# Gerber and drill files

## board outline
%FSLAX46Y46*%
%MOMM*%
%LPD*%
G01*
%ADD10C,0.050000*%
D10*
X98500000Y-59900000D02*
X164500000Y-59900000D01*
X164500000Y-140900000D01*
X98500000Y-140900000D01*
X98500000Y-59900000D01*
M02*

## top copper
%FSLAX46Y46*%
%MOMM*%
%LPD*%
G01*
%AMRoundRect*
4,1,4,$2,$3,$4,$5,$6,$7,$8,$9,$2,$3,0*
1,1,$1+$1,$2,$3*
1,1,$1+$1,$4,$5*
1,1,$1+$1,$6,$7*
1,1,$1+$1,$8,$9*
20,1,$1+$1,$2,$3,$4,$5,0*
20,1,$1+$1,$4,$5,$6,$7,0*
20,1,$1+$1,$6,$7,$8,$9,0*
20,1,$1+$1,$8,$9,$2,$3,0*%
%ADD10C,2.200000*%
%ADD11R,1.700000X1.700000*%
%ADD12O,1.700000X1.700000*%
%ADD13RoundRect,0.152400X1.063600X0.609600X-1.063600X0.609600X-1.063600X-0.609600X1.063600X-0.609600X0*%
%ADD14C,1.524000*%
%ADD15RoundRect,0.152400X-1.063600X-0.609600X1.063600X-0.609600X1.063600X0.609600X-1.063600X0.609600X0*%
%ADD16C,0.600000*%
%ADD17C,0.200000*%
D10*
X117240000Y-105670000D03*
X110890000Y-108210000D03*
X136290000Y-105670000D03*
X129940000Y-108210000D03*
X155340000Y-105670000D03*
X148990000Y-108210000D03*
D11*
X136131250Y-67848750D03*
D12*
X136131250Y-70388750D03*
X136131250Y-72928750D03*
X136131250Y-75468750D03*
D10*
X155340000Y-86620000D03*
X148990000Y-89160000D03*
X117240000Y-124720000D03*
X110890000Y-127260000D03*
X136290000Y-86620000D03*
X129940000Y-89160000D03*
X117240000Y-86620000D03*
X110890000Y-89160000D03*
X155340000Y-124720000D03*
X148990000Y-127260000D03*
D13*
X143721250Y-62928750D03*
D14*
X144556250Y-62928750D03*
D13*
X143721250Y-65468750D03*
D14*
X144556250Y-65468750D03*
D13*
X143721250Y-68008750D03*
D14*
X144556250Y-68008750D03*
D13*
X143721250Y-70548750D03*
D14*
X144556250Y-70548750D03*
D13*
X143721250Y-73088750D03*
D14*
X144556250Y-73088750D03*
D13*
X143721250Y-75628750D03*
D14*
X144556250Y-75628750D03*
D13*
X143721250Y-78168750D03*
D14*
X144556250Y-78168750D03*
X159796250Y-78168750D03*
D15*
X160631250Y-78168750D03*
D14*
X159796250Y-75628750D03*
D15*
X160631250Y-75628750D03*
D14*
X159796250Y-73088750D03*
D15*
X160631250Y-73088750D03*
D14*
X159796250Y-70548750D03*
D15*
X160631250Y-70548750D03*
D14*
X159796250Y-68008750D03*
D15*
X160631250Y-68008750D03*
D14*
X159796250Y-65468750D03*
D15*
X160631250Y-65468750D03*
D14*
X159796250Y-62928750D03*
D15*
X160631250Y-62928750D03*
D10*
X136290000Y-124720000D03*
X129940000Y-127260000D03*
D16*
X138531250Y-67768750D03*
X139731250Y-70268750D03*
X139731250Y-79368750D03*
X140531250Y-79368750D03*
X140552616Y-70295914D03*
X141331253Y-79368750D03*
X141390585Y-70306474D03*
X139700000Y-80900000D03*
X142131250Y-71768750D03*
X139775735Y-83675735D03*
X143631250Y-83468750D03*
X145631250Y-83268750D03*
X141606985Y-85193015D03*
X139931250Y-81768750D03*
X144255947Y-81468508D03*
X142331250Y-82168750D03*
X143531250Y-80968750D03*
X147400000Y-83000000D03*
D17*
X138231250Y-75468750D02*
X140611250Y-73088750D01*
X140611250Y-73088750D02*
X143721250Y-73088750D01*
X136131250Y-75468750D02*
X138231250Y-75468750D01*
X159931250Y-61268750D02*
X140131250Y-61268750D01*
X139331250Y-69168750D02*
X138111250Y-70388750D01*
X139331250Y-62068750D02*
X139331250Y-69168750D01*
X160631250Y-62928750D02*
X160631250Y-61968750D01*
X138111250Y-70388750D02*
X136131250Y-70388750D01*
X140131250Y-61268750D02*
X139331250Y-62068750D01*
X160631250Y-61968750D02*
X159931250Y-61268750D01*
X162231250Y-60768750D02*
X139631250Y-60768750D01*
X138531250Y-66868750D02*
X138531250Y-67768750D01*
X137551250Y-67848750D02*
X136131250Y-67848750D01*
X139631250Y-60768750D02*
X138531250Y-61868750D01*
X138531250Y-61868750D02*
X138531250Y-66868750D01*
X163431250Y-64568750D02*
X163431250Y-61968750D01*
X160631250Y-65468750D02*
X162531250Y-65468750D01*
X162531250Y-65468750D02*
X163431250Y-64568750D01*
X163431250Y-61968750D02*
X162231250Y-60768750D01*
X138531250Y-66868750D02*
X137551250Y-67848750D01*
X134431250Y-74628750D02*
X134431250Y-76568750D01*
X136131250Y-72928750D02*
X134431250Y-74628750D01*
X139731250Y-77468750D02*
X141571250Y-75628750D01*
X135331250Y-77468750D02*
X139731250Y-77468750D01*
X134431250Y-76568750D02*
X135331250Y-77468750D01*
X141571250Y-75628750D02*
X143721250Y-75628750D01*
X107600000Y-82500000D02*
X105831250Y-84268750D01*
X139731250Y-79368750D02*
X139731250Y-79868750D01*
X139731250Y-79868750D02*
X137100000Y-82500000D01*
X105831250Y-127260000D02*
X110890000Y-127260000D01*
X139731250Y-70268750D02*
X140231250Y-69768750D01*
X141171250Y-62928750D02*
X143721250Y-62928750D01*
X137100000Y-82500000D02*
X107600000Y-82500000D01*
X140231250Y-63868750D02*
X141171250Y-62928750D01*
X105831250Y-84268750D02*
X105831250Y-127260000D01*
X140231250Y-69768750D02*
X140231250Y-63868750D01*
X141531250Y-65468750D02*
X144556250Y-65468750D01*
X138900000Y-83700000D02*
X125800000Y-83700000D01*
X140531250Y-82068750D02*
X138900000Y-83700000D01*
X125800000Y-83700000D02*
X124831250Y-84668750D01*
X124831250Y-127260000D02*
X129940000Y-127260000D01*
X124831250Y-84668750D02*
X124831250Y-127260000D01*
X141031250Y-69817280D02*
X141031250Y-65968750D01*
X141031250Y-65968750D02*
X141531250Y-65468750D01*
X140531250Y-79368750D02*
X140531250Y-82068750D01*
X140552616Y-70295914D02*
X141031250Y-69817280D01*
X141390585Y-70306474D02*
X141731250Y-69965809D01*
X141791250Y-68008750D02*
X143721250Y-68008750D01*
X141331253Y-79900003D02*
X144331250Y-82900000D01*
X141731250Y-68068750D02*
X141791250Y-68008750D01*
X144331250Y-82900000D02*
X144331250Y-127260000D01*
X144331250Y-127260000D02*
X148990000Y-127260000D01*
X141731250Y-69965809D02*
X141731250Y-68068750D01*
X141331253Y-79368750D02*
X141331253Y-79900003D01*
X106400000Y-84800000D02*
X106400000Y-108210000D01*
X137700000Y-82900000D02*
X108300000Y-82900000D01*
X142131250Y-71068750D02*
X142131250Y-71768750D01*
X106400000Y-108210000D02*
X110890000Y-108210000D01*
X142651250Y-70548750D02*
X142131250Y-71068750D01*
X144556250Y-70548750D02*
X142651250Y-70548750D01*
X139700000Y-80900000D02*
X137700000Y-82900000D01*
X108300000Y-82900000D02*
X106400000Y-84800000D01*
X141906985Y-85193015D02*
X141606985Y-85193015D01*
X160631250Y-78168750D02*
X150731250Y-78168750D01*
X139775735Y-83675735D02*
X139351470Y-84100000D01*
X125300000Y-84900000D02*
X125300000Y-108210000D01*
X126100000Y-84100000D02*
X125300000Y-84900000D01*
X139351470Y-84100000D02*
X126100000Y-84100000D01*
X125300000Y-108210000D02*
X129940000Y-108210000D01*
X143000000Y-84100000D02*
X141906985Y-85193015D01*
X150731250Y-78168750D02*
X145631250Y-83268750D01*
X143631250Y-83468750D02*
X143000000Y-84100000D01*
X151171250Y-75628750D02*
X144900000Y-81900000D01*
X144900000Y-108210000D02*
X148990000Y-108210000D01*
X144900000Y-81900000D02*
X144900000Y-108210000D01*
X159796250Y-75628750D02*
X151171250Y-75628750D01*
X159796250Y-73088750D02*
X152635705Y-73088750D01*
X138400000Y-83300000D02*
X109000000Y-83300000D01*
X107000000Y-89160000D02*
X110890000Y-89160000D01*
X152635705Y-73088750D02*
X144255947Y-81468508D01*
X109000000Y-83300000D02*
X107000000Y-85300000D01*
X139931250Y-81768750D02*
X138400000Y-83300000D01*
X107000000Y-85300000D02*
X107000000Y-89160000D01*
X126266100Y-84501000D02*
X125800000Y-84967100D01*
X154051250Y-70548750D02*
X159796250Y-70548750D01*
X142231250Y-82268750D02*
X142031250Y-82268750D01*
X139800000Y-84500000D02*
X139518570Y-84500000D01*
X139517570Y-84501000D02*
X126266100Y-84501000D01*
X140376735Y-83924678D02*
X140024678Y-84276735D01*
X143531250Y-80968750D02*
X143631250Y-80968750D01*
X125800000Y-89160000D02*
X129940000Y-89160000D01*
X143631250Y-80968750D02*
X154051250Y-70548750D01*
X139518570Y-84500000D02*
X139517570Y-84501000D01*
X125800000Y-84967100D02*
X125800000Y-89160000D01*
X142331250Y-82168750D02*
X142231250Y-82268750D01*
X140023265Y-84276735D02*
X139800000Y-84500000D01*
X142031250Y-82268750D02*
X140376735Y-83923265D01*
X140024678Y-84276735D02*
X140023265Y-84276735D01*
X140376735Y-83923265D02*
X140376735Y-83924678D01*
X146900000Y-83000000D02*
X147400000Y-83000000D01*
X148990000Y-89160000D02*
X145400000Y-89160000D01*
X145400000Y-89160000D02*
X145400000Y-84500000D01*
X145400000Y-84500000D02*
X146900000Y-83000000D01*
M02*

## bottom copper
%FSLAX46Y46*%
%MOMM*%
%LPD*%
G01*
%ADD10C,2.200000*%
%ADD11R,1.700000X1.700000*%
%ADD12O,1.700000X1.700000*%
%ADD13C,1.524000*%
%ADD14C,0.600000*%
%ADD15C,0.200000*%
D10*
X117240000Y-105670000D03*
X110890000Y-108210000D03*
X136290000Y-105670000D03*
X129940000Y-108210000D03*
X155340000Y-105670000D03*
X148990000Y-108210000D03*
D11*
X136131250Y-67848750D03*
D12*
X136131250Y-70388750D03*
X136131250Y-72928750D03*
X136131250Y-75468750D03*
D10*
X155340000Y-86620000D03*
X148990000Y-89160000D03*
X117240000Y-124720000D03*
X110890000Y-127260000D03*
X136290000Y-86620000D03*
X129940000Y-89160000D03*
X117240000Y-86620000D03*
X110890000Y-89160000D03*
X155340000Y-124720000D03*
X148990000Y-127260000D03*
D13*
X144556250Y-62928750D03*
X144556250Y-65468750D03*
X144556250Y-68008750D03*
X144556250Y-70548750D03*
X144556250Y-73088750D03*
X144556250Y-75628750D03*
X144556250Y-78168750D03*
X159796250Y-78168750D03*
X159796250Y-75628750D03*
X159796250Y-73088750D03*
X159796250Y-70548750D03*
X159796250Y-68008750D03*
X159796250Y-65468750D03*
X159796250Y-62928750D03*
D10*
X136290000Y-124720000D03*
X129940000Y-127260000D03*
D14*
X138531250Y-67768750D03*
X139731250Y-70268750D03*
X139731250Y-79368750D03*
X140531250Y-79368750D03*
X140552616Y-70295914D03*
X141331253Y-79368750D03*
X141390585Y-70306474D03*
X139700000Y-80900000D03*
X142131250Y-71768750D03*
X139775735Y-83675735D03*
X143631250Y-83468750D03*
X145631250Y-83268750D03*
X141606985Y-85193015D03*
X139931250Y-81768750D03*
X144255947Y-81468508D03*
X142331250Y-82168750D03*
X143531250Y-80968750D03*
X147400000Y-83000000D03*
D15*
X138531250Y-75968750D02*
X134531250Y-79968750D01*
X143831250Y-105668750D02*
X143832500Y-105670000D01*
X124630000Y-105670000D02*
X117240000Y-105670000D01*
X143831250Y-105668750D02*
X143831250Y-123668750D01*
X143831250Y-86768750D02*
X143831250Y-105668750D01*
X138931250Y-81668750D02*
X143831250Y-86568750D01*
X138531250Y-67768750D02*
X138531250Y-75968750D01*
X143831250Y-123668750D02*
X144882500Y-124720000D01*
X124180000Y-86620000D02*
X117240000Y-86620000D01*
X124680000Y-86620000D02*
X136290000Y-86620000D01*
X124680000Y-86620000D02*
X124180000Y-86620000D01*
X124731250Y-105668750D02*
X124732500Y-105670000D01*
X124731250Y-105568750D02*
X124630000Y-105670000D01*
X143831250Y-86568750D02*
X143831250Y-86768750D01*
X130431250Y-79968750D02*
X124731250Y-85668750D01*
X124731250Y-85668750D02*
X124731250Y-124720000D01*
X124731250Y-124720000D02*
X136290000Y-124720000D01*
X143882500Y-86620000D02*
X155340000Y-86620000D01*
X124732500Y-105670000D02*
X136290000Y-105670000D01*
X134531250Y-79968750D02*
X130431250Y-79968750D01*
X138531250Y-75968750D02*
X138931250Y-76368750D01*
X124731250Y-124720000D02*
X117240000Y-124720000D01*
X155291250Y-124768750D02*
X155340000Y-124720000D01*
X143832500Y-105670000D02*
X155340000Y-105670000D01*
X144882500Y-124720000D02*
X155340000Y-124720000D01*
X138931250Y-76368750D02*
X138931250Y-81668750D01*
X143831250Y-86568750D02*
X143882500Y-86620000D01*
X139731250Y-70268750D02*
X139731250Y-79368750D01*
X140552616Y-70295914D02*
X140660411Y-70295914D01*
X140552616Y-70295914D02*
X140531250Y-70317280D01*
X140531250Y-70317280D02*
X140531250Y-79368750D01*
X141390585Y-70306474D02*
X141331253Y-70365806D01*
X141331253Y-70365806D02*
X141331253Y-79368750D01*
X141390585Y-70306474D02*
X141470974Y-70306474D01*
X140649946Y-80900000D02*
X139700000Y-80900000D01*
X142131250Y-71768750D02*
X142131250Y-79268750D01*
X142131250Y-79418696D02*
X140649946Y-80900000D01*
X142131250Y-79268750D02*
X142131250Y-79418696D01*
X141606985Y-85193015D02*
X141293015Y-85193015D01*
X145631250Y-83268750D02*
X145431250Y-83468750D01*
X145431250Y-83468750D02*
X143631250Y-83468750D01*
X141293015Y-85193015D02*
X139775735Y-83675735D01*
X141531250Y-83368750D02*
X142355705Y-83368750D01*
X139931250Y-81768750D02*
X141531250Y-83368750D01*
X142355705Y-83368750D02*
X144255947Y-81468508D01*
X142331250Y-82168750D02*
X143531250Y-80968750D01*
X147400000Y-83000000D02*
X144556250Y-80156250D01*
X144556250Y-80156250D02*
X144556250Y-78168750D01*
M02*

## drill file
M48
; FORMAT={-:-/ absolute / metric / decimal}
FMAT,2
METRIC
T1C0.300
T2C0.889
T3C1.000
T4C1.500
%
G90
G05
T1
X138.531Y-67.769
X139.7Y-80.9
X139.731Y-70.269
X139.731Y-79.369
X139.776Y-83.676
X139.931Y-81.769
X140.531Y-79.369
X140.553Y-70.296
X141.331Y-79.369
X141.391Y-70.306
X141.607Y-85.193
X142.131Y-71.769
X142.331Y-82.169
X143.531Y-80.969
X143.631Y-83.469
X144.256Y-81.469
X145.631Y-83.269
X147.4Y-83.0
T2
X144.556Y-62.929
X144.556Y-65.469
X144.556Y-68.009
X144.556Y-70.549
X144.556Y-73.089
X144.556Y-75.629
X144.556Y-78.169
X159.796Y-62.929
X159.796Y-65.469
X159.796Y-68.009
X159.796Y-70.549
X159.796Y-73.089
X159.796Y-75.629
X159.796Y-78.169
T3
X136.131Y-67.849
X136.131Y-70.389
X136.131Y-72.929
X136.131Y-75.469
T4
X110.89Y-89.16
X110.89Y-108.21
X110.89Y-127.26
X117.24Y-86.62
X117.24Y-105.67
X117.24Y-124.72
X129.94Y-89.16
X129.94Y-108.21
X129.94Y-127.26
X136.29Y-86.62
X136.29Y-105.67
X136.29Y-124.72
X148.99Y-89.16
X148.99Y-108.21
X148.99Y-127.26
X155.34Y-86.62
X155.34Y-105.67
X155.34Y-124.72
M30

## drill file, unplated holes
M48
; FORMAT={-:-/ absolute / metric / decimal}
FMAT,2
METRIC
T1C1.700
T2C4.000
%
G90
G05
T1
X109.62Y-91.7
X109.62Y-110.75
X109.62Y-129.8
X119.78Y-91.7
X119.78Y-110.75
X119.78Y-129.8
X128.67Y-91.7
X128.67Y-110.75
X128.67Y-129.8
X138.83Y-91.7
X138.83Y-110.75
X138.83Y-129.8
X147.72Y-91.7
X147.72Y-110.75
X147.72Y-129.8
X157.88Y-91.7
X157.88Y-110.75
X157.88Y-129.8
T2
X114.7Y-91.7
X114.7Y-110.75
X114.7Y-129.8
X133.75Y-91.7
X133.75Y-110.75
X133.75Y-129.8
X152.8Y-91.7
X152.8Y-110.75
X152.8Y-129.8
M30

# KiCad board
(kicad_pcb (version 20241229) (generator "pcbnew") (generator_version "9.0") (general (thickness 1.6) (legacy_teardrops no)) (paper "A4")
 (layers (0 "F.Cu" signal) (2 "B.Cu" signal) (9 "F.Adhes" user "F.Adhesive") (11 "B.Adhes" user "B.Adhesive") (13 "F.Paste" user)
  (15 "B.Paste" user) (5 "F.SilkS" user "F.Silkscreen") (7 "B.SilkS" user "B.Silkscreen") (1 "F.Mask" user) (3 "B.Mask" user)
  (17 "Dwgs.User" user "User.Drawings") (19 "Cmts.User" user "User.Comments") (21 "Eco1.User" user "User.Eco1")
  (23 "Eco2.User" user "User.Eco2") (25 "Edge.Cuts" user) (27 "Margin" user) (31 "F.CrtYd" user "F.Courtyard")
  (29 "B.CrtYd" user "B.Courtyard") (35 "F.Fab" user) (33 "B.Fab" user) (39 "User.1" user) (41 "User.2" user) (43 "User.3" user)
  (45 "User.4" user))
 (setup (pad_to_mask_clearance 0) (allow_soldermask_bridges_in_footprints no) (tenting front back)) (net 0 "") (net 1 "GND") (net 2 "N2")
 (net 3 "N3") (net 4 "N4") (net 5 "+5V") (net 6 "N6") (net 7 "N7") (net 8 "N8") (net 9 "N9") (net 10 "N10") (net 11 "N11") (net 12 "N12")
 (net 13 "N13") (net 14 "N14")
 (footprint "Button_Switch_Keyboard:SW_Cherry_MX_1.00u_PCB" (layer "F.Cu") (at 117.24 105.67)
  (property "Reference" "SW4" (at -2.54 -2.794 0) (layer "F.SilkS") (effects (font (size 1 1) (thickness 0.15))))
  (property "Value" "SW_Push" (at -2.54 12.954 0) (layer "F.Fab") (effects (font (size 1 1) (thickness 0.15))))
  (pad "" np_thru_hole circle (at -7.62 5.08) (size 1.7 1.7) (drill 1.7) (layers "*.Cu" "*.Mask"))
  (pad "" np_thru_hole circle (at -2.54 5.08) (size 4 4) (drill 4) (layers "*.Cu" "*.Mask"))
  (pad "" np_thru_hole circle (at 2.54 5.08) (size 1.7 1.7) (drill 1.7) (layers "*.Cu" "*.Mask"))
  (pad "1" thru_hole circle (at 0 0) (size 2.2 2.2) (drill 1.5) (layers "*.Cu" "*.Mask") (remove_unused_layers no) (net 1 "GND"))
  (pad "2" thru_hole circle (at -6.35 2.54) (size 2.2 2.2) (drill 1.5) (layers "*.Cu" "*.Mask") (remove_unused_layers no) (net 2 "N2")))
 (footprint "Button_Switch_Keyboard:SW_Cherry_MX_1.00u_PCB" (layer "F.Cu") (at 136.29 105.67)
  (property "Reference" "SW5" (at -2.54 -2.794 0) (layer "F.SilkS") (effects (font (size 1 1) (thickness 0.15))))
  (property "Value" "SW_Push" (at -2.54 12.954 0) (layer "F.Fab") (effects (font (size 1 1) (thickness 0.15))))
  (pad "" np_thru_hole circle (at -7.62 5.08) (size 1.7 1.7) (drill 1.7) (layers "*.Cu" "*.Mask"))
  (pad "" np_thru_hole circle (at -2.54 5.08) (size 4 4) (drill 4) (layers "*.Cu" "*.Mask"))
  (pad "" np_thru_hole circle (at 2.54 5.08) (size 1.7 1.7) (drill 1.7) (layers "*.Cu" "*.Mask"))
  (pad "1" thru_hole circle (at 0 0) (size 2.2 2.2) (drill 1.5) (layers "*.Cu" "*.Mask") (remove_unused_layers no) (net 1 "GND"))
  (pad "2" thru_hole circle (at -6.35 2.54) (size 2.2 2.2) (drill 1.5) (layers "*.Cu" "*.Mask") (remove_unused_layers no) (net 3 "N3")))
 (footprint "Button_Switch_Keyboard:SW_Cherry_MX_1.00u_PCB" (layer "F.Cu") (at 155.34 105.67)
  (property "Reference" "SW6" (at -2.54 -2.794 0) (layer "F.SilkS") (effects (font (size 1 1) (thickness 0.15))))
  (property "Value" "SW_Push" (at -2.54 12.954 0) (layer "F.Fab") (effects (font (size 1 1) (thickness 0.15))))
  (pad "" np_thru_hole circle (at -7.62 5.08) (size 1.7 1.7) (drill 1.7) (layers "*.Cu" "*.Mask"))
  (pad "" np_thru_hole circle (at -2.54 5.08) (size 4 4) (drill 4) (layers "*.Cu" "*.Mask"))
  (pad "" np_thru_hole circle (at 2.54 5.08) (size 1.7 1.7) (drill 1.7) (layers "*.Cu" "*.Mask"))
  (pad "1" thru_hole circle (at 0 0) (size 2.2 2.2) (drill 1.5) (layers "*.Cu" "*.Mask") (remove_unused_layers no) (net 1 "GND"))
  (pad "2" thru_hole circle (at -6.35 2.54) (size 2.2 2.2) (drill 1.5) (layers "*.Cu" "*.Mask") (remove_unused_layers no) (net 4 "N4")))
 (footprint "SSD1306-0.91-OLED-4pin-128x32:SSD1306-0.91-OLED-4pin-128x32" (layer "F.Cu") (at 99.63125 65.65875)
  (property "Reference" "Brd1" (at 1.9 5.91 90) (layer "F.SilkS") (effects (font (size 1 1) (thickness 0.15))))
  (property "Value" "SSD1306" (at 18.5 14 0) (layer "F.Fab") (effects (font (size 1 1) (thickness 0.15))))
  (pad "1" thru_hole rect (at 36.5 2.19) (size 1.7 1.7) (drill 1) (layers "*.Cu" "*.Mask") (remove_unused_layers no) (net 1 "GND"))
  (pad "2" thru_hole oval (at 36.5 4.73) (size 1.7 1.7) (drill 1) (layers "*.Cu" "*.Mask") (remove_unused_layers no) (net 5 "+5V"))
  (pad "3" thru_hole oval (at 36.5 7.27) (size 1.7 1.7) (drill 1) (layers "*.Cu" "*.Mask") (remove_unused_layers no) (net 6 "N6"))
  (pad "4" thru_hole oval (at 36.5 9.81) (size 1.7 1.7) (drill 1) (layers "*.Cu" "*.Mask") (remove_unused_layers no) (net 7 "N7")))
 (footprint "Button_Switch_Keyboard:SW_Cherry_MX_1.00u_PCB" (layer "F.Cu") (at 155.34 86.62)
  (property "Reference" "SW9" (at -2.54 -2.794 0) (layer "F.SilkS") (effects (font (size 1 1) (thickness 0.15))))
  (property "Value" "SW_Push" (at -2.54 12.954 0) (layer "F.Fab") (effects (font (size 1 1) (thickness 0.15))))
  (pad "" np_thru_hole circle (at -7.62 5.08) (size 1.7 1.7) (drill 1.7) (layers "*.Cu" "*.Mask"))
  (pad "" np_thru_hole circle (at -2.54 5.08) (size 4 4) (drill 4) (layers "*.Cu" "*.Mask"))
  (pad "" np_thru_hole circle (at 2.54 5.08) (size 1.7 1.7) (drill 1.7) (layers "*.Cu" "*.Mask"))
  (pad "1" thru_hole circle (at 0 0) (size 2.2 2.2) (drill 1.5) (layers "*.Cu" "*.Mask") (remove_unused_layers no) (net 1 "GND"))
  (pad "2" thru_hole circle (at -6.35 2.54) (size 2.2 2.2) (drill 1.5) (layers "*.Cu" "*.Mask") (remove_unused_layers no) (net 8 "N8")))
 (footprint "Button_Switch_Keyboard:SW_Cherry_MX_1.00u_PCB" (layer "F.Cu") (at 117.24 124.72)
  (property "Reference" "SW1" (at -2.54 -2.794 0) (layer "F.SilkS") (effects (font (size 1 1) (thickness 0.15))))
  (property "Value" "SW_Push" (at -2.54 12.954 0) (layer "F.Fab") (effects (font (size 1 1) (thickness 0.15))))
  (pad "" np_thru_hole circle (at -7.62 5.08) (size 1.7 1.7) (drill 1.7) (layers "*.Cu" "*.Mask"))
  (pad "" np_thru_hole circle (at -2.54 5.08) (size 4 4) (drill 4) (layers "*.Cu" "*.Mask"))
  (pad "" np_thru_hole circle (at 2.54 5.08) (size 1.7 1.7) (drill 1.7) (layers "*.Cu" "*.Mask"))
  (pad "1" thru_hole circle (at 0 0) (size 2.2 2.2) (drill 1.5) (layers "*.Cu" "*.Mask") (remove_unused_layers no) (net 1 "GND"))
  (pad "2" thru_hole circle (at -6.35 2.54) (size 2.2 2.2) (drill 1.5) (layers "*.Cu" "*.Mask") (remove_unused_layers no) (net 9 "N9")))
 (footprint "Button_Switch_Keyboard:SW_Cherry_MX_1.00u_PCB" (layer "F.Cu") (at 136.29 86.62)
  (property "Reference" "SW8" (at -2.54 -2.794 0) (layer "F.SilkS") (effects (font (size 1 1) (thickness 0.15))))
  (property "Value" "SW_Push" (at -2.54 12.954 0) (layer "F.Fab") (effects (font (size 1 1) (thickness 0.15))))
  (pad "" np_thru_hole circle (at -7.62 5.08) (size 1.7 1.7) (drill 1.7) (layers "*.Cu" "*.Mask"))
  (pad "" np_thru_hole circle (at -2.54 5.08) (size 4 4) (drill 4) (layers "*.Cu" "*.Mask"))
  (pad "" np_thru_hole circle (at 2.54 5.08) (size 1.7 1.7) (drill 1.7) (layers "*.Cu" "*.Mask"))
  (pad "1" thru_hole circle (at 0 0) (size 2.2 2.2) (drill 1.5) (layers "*.Cu" "*.Mask") (remove_unused_layers no) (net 1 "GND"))
  (pad "2" thru_hole circle (at -6.35 2.54) (size 2.2 2.2) (drill 1.5) (layers "*.Cu" "*.Mask") (remove_unused_layers no) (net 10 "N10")))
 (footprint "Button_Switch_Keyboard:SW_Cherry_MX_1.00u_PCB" (layer "F.Cu") (at 117.24 86.62)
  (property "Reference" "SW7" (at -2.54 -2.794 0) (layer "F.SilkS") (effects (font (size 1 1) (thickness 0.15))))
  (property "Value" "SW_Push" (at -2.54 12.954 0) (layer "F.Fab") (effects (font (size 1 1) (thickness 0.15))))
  (pad "" np_thru_hole circle (at -7.62 5.08) (size 1.7 1.7) (drill 1.7) (layers "*.Cu" "*.Mask"))
  (pad "" np_thru_hole circle (at -2.54 5.08) (size 4 4) (drill 4) (layers "*.Cu" "*.Mask"))
  (pad "" np_thru_hole circle (at 2.54 5.08) (size 1.7 1.7) (drill 1.7) (layers "*.Cu" "*.Mask"))
  (pad "1" thru_hole circle (at 0 0) (size 2.2 2.2) (drill 1.5) (layers "*.Cu" "*.Mask") (remove_unused_layers no) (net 1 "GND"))
  (pad "2" thru_hole circle (at -6.35 2.54) (size 2.2 2.2) (drill 1.5) (layers "*.Cu" "*.Mask") (remove_unused_layers no) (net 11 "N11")))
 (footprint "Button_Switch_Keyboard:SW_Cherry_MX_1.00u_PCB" (layer "F.Cu") (at 155.34 124.72)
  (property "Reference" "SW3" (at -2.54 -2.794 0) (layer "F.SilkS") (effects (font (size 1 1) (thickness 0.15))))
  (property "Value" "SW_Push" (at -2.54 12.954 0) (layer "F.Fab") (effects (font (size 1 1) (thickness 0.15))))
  (pad "" np_thru_hole circle (at -7.62 5.08) (size 1.7 1.7) (drill 1.7) (layers "*.Cu" "*.Mask"))
  (pad "" np_thru_hole circle (at -2.54 5.08) (size 4 4) (drill 4) (layers "*.Cu" "*.Mask"))
  (pad "" np_thru_hole circle (at 2.54 5.08) (size 1.7 1.7) (drill 1.7) (layers "*.Cu" "*.Mask"))
  (pad "1" thru_hole circle (at 0 0) (size 2.2 2.2) (drill 1.5) (layers "*.Cu" "*.Mask") (remove_unused_layers no) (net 1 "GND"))
  (pad "2" thru_hole circle (at -6.35 2.54) (size 2.2 2.2) (drill 1.5) (layers "*.Cu" "*.Mask") (remove_unused_layers no) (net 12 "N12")))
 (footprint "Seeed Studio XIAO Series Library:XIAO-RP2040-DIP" (layer "F.Cu") (at 152.17625 70.54875)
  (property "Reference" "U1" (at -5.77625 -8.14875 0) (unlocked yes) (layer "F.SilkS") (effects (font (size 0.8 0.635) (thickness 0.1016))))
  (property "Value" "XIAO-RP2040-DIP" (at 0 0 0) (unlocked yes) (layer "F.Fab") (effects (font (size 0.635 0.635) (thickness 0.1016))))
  (pad "1" smd roundrect (at -8.455 -7.62 180) (size 2.432 1.524) (layers "F.Cu" "F.Mask") (roundrect_rratio 0.1) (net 9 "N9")
   (thermal_bridge_angle 45))
  (pad "1" thru_hole circle (at -7.62 -7.62 180) (size 1.524 1.524) (drill 0.889) (layers "*.Cu" "*.Mask") (remove_unused_layers no)
   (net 9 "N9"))
  (pad "2" smd roundrect (at -8.455 -5.08 180) (size 2.432 1.524) (layers "F.Cu" "F.Mask") (roundrect_rratio 0.1) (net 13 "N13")
   (thermal_bridge_angle 45))
  (pad "2" thru_hole circle (at -7.62 -5.08 180) (size 1.524 1.524) (drill 0.889) (layers "*.Cu" "*.Mask") (remove_unused_layers no)
   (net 13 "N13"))
  (pad "3" smd roundrect (at -8.455 -2.54 180) (size 2.432 1.524) (layers "F.Cu" "F.Mask") (roundrect_rratio 0.1) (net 12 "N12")
   (thermal_bridge_angle 45))
  (pad "3" thru_hole circle (at -7.62 -2.54 180) (size 1.524 1.524) (drill 0.889) (layers "*.Cu" "*.Mask") (remove_unused_layers no)
   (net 12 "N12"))
  (pad "4" smd roundrect (at -8.455 0 180) (size 2.432 1.524) (layers "F.Cu" "F.Mask") (roundrect_rratio 0.1) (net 2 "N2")
   (thermal_bridge_angle 45))
  (pad "4" thru_hole circle (at -7.62 0 180) (size 1.524 1.524) (drill 0.889) (layers "*.Cu" "*.Mask") (remove_unused_layers no)
   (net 2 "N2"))
  (pad "5" smd roundrect (at -8.455 2.54 180) (size 2.432 1.524) (layers "F.Cu" "F.Mask") (roundrect_rratio 0.1) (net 7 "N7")
   (thermal_bridge_angle 45))
  (pad "5" thru_hole circle (at -7.62 2.54 180) (size 1.524 1.524) (drill 0.889) (layers "*.Cu" "*.Mask") (remove_unused_layers no)
   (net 7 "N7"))
  (pad "6" smd roundrect (at -8.455 5.08 180) (size 2.432 1.524) (layers "F.Cu" "F.Mask") (roundrect_rratio 0.1) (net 6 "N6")
   (thermal_bridge_angle 45))
  (pad "6" thru_hole circle (at -7.62 5.08 180) (size 1.524 1.524) (drill 0.889) (layers "*.Cu" "*.Mask") (remove_unused_layers no)
   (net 6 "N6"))
  (pad "7" smd roundrect (at -8.455 7.62 180) (size 2.432 1.524) (layers "F.Cu" "F.Mask") (roundrect_rratio 0.1) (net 8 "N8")
   (thermal_bridge_angle 45))
  (pad "7" thru_hole circle (at -7.62 7.62 180) (size 1.524 1.524) (drill 0.889) (layers "*.Cu" "*.Mask") (remove_unused_layers no)
   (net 8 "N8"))
  (pad "8" thru_hole circle (at 7.62 7.62) (size 1.524 1.524) (drill 0.889) (layers "*.Cu" "*.Mask") (remove_unused_layers no) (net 3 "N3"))
  (pad "8" smd roundrect (at 8.455 7.62) (size 2.432 1.524) (layers "F.Cu" "F.Mask") (roundrect_rratio 0.1) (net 3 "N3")
   (thermal_bridge_angle 45))
  (pad "9" thru_hole circle (at 7.62 5.08) (size 1.524 1.524) (drill 0.889) (layers "*.Cu" "*.Mask") (remove_unused_layers no) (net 4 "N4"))
  (pad "9" smd roundrect (at 8.455 5.08) (size 2.432 1.524) (layers "F.Cu" "F.Mask") (roundrect_rratio 0.1) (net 4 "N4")
   (thermal_bridge_angle 45))
  (pad "10" thru_hole circle (at 7.62 2.54) (size 1.524 1.524) (drill 0.889) (layers "*.Cu" "*.Mask") (remove_unused_layers no)
   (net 11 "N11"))
  (pad "10" smd roundrect (at 8.455 2.54) (size 2.432 1.524) (layers "F.Cu" "F.Mask") (roundrect_rratio 0.1) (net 11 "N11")
   (thermal_bridge_angle 45))
  (pad "11" thru_hole circle (at 7.62 0) (size 1.524 1.524) (drill 0.889) (layers "*.Cu" "*.Mask") (remove_unused_layers no) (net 10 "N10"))
  (pad "11" smd roundrect (at 8.455 0) (size 2.432 1.524) (layers "F.Cu" "F.Mask") (roundrect_rratio 0.1) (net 10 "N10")
   (thermal_bridge_angle 45))
  (pad "12" thru_hole circle (at 7.62 -2.54) (size 1.524 1.524) (drill 0.889) (layers "*.Cu" "*.Mask") (remove_unused_layers no)
   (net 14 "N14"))
  (pad "12" smd roundrect (at 8.455 -2.54) (size 2.432 1.524) (layers "F.Cu" "F.Mask") (roundrect_rratio 0.1) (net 14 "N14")
   (thermal_bridge_angle 45))
  (pad "13" thru_hole circle (at 7.62 -5.08) (size 1.524 1.524) (drill 0.889) (layers "*.Cu" "*.Mask") (remove_unused_layers no)
   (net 1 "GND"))
  (pad "13" smd roundrect (at 8.455 -5.08) (size 2.432 1.524) (layers "F.Cu" "F.Mask") (roundrect_rratio 0.1) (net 1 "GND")
   (thermal_bridge_angle 45))
  (pad "14" thru_hole circle (at 7.62 -7.62) (size 1.524 1.524) (drill 0.889) (layers "*.Cu" "*.Mask") (remove_unused_layers no)
   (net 5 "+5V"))
  (pad "14" smd roundrect (at 8.455 -7.62) (size 2.432 1.524) (layers "F.Cu" "F.Mask") (roundrect_rratio 0.1) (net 5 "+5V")
   (thermal_bridge_angle 45)))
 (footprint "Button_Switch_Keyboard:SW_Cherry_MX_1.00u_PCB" (layer "F.Cu") (at 136.29 124.72)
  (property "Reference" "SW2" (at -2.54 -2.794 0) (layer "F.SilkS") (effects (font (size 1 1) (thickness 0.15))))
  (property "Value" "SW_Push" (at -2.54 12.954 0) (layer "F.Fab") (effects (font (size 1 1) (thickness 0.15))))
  (pad "" np_thru_hole circle (at -7.62 5.08) (size 1.7 1.7) (drill 1.7) (layers "*.Cu" "*.Mask"))
  (pad "" np_thru_hole circle (at -2.54 5.08) (size 4 4) (drill 4) (layers "*.Cu" "*.Mask"))
  (pad "" np_thru_hole circle (at 2.54 5.08) (size 1.7 1.7) (drill 1.7) (layers "*.Cu" "*.Mask"))
  (pad "1" thru_hole circle (at 0 0) (size 2.2 2.2) (drill 1.5) (layers "*.Cu" "*.Mask") (remove_unused_layers no) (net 1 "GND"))
  (pad "2" thru_hole circle (at -6.35 2.54) (size 2.2 2.2) (drill 1.5) (layers "*.Cu" "*.Mask") (remove_unused_layers no) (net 13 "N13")))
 (gr_rect (start 98.5 59.9) (end 164.5 140.9) (stroke (width 0.05) (type solid)) (fill no) (layer "Edge.Cuts"))
 (segment (start 138.23125 75.46875) (end 140.61125 73.08875) (width 0.2) (layer "F.Cu") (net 7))
 (segment (start 140.61125 73.08875) (end 143.72125 73.08875) (width 0.2) (layer "F.Cu") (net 7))
 (segment (start 136.13125 75.46875) (end 138.23125 75.46875) (width 0.2) (layer "F.Cu") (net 7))
 (segment (start 159.93125 61.26875) (end 140.13125 61.26875) (width 0.2) (layer "F.Cu") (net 5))
 (segment (start 139.33125 69.16875) (end 138.11125 70.38875) (width 0.2) (layer "F.Cu") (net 5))
 (segment (start 139.33125 62.06875) (end 139.33125 69.16875) (width 0.2) (layer "F.Cu") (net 5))
 (segment (start 160.63125 62.92875) (end 160.63125 61.96875) (width 0.2) (layer "F.Cu") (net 5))
 (segment (start 138.11125 70.38875) (end 136.13125 70.38875) (width 0.2) (layer "F.Cu") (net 5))
 (segment (start 140.13125 61.26875) (end 139.33125 62.06875) (width 0.2) (layer "F.Cu") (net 5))
 (segment (start 160.63125 61.96875) (end 159.93125 61.26875) (width 0.2) (layer "F.Cu") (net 5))
 (segment (start 162.23125 60.76875) (end 139.63125 60.76875) (width 0.2) (layer "F.Cu") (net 1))
 (segment (start 138.53125 66.86875) (end 138.53125 67.76875) (width 0.2) (layer "F.Cu") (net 1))
 (segment (start 137.55125 67.84875) (end 136.13125 67.84875) (width 0.2) (layer "F.Cu") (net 1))
 (segment (start 139.63125 60.76875) (end 138.53125 61.86875) (width 0.2) (layer "F.Cu") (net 1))
 (segment (start 138.53125 61.86875) (end 138.53125 66.86875) (width 0.2) (layer "F.Cu") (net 1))
 (segment (start 163.43125 64.56875) (end 163.43125 61.96875) (width 0.2) (layer "F.Cu") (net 1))
 (segment (start 160.63125 65.46875) (end 162.53125 65.46875) (width 0.2) (layer "F.Cu") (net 1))
 (segment (start 162.53125 65.46875) (end 163.43125 64.56875) (width 0.2) (layer "F.Cu") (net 1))
 (segment (start 163.43125 61.96875) (end 162.23125 60.76875) (width 0.2) (layer "F.Cu") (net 1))
 (segment (start 138.53125 66.86875) (end 137.55125 67.84875) (width 0.2) (layer "F.Cu") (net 1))
 (via (at 138.53125 67.76875) (size 0.6) (drill 0.3) (layers "F.Cu" "B.Cu") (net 1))
 (segment (start 138.53125 75.96875) (end 134.53125 79.96875) (width 0.2) (layer "B.Cu") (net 1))
 (segment (start 143.83125 105.66875) (end 143.8325 105.67) (width 0.2) (layer "B.Cu") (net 1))
 (segment (start 124.63 105.67) (end 117.24 105.67) (width 0.2) (layer "B.Cu") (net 1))
 (segment (start 143.83125 105.66875) (end 143.83125 123.66875) (width 0.2) (layer "B.Cu") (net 1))
 (segment (start 143.83125 86.76875) (end 143.83125 105.66875) (width 0.2) (layer "B.Cu") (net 1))
 (segment (start 138.93125 81.66875) (end 143.83125 86.56875) (width 0.2) (layer "B.Cu") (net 1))
 (segment (start 138.53125 67.76875) (end 138.53125 75.96875) (width 0.2) (layer "B.Cu") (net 1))
 (segment (start 143.83125 123.66875) (end 144.8825 124.72) (width 0.2) (layer "B.Cu") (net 1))
 (segment (start 124.18 86.62) (end 117.24 86.62) (width 0.2) (layer "B.Cu") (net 1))
 (segment (start 124.68 86.62) (end 136.29 86.62) (width 0.2) (layer "B.Cu") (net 1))
 (segment (start 124.68 86.62) (end 124.18 86.62) (width 0.2) (layer "B.Cu") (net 1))
 (segment (start 124.73125 105.66875) (end 124.7325 105.67) (width 0.2) (layer "B.Cu") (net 1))
 (segment (start 124.73125 105.56875) (end 124.63 105.67) (width 0.2) (layer "B.Cu") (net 1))
 (segment (start 143.83125 86.56875) (end 143.83125 86.76875) (width 0.2) (layer "B.Cu") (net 1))
 (segment (start 130.43125 79.96875) (end 124.73125 85.66875) (width 0.2) (layer "B.Cu") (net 1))
 (segment (start 124.73125 85.66875) (end 124.73125 124.72) (width 0.2) (layer "B.Cu") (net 1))
 (segment (start 124.73125 124.72) (end 136.29 124.72) (width 0.2) (layer "B.Cu") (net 1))
 (segment (start 143.8825 86.62) (end 155.34 86.62) (width 0.2) (layer "B.Cu") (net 1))
 (segment (start 124.7325 105.67) (end 136.29 105.67) (width 0.2) (layer "B.Cu") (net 1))
 (segment (start 134.53125 79.96875) (end 130.43125 79.96875) (width 0.2) (layer "B.Cu") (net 1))
 (segment (start 138.53125 75.96875) (end 138.93125 76.36875) (width 0.2) (layer "B.Cu") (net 1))
 (segment (start 124.73125 124.72) (end 117.24 124.72) (width 0.2) (layer "B.Cu") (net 1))
 (segment (start 155.29125 124.76875) (end 155.34 124.72) (width 0.2) (layer "B.Cu") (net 1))
 (segment (start 143.8325 105.67) (end 155.34 105.67) (width 0.2) (layer "B.Cu") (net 1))
 (segment (start 144.8825 124.72) (end 155.34 124.72) (width 0.2) (layer "B.Cu") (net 1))
 (segment (start 138.93125 76.36875) (end 138.93125 81.66875) (width 0.2) (layer "B.Cu") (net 1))
 (segment (start 143.83125 86.56875) (end 143.8825 86.62) (width 0.2) (layer "B.Cu") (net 1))
 (segment (start 134.43125 74.62875) (end 134.43125 76.56875) (width 0.2) (layer "F.Cu") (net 6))
 (segment (start 136.13125 72.92875) (end 134.43125 74.62875) (width 0.2) (layer "F.Cu") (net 6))
 (segment (start 139.73125 77.46875) (end 141.57125 75.62875) (width 0.2) (layer "F.Cu") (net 6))
 (segment (start 135.33125 77.46875) (end 139.73125 77.46875) (width 0.2) (layer "F.Cu") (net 6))
 (segment (start 134.43125 76.56875) (end 135.33125 77.46875) (width 0.2) (layer "F.Cu") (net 6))
 (segment (start 141.57125 75.62875) (end 143.72125 75.62875) (width 0.2) (layer "F.Cu") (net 6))
 (segment (start 107.6 82.5) (end 105.83125 84.26875) (width 0.2) (layer "F.Cu") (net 9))
 (segment (start 139.73125 79.36875) (end 139.73125 79.86875) (width 0.2) (layer "F.Cu") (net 9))
 (segment (start 139.73125 79.86875) (end 137.1 82.5) (width 0.2) (layer "F.Cu") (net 9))
 (segment (start 105.83125 127.26) (end 110.89 127.26) (width 0.2) (layer "F.Cu") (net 9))
 (segment (start 139.73125 70.26875) (end 140.23125 69.76875) (width 0.2) (layer "F.Cu") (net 9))
 (segment (start 141.17125 62.92875) (end 143.72125 62.92875) (width 0.2) (layer "F.Cu") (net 9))
 (segment (start 137.1 82.5) (end 107.6 82.5) (width 0.2) (layer "F.Cu") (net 9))
 (segment (start 140.23125 63.86875) (end 141.17125 62.92875) (width 0.2) (layer "F.Cu") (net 9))
 (segment (start 105.83125 84.26875) (end 105.83125 127.26) (width 0.2) (layer "F.Cu") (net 9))
 (segment (start 140.23125 69.76875) (end 140.23125 63.86875) (width 0.2) (layer "F.Cu") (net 9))
 (via (at 139.73125 70.26875) (size 0.6) (drill 0.3) (layers "F.Cu" "B.Cu") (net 9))
 (via (at 139.73125 79.36875) (size 0.6) (drill 0.3) (layers "F.Cu" "B.Cu") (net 9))
 (segment (start 139.73125 70.26875) (end 139.73125 79.36875) (width 0.2) (layer "B.Cu") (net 9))
 (segment (start 141.53125 65.46875) (end 144.55625 65.46875) (width 0.2) (layer "F.Cu") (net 13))
 (segment (start 138.9 83.7) (end 125.8 83.7) (width 0.2) (layer "F.Cu") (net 13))
 (segment (start 140.53125 82.06875) (end 138.9 83.7) (width 0.2) (layer "F.Cu") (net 13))
 (segment (start 125.8 83.7) (end 124.83125 84.66875) (width 0.2) (layer "F.Cu") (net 13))
 (segment (start 124.83125 127.26) (end 129.94 127.26) (width 0.2) (layer "F.Cu") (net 13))
 (segment (start 124.83125 84.66875) (end 124.83125 127.26) (width 0.2) (layer "F.Cu") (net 13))
 (segment (start 141.03125 69.81728) (end 141.03125 65.96875) (width 0.2) (layer "F.Cu") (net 13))
 (segment (start 141.03125 65.96875) (end 141.53125 65.46875) (width 0.2) (layer "F.Cu") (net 13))
 (segment (start 140.53125 79.36875) (end 140.53125 82.06875) (width 0.2) (layer "F.Cu") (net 13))
 (segment (start 140.552616 70.295914) (end 141.03125 69.81728) (width 0.2) (layer "F.Cu") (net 13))
 (via (at 140.53125 79.36875) (size 0.6) (drill 0.3) (layers "F.Cu" "B.Cu") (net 13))
 (via (at 140.552616 70.295914) (size 0.6) (drill 0.3) (layers "F.Cu" "B.Cu") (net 13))
 (segment (start 140.552616 70.295914) (end 140.660411 70.295914) (width 0.2) (layer "B.Cu") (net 13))
 (segment (start 140.552616 70.295914) (end 140.53125 70.31728) (width 0.2) (layer "B.Cu") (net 13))
 (segment (start 140.53125 70.31728) (end 140.53125 79.36875) (width 0.2) (layer "B.Cu") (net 13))
 (segment (start 141.390585 70.306474) (end 141.73125 69.965809) (width 0.2) (layer "F.Cu") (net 12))
 (segment (start 141.79125 68.00875) (end 143.72125 68.00875) (width 0.2) (layer "F.Cu") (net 12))
 (segment (start 141.331253 79.900003) (end 144.33125 82.9) (width 0.2) (layer "F.Cu") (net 12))
 (segment (start 141.73125 68.06875) (end 141.79125 68.00875) (width 0.2) (layer "F.Cu") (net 12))
 (segment (start 144.33125 82.9) (end 144.33125 127.26) (width 0.2) (layer "F.Cu") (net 12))
 (segment (start 144.33125 127.26) (end 148.99 127.26) (width 0.2) (layer "F.Cu") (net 12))
 (segment (start 141.73125 69.965809) (end 141.73125 68.06875) (width 0.2) (layer "F.Cu") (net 12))
 (segment (start 141.331253 79.36875) (end 141.331253 79.900003) (width 0.2) (layer "F.Cu") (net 12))
 (via (at 141.331253 79.36875) (size 0.6) (drill 0.3) (layers "F.Cu" "B.Cu") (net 12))
 (via (at 141.390585 70.306474) (size 0.6) (drill 0.3) (layers "F.Cu" "B.Cu") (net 12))
 (segment (start 141.390585 70.306474) (end 141.331253 70.365806) (width 0.2) (layer "B.Cu") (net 12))
 (segment (start 141.331253 70.365806) (end 141.331253 79.36875) (width 0.2) (layer "B.Cu") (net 12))
 (segment (start 141.390585 70.306474) (end 141.470974 70.306474) (width 0.2) (layer "B.Cu") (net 12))
 (segment (start 106.4 84.8) (end 106.4 108.21) (width 0.2) (layer "F.Cu") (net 2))
 (segment (start 137.7 82.9) (end 108.3 82.9) (width 0.2) (layer "F.Cu") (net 2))
 (segment (start 142.13125 71.06875) (end 142.13125 71.76875) (width 0.2) (layer "F.Cu") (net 2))
 (segment (start 106.4 108.21) (end 110.89 108.21) (width 0.2) (layer "F.Cu") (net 2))
 (segment (start 142.65125 70.54875) (end 142.13125 71.06875) (width 0.2) (layer "F.Cu") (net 2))
 (segment (start 144.55625 70.54875) (end 142.65125 70.54875) (width 0.2) (layer "F.Cu") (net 2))
 (segment (start 139.7 80.9) (end 137.7 82.9) (width 0.2) (layer "F.Cu") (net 2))
 (segment (start 108.3 82.9) (end 106.4 84.8) (width 0.2) (layer "F.Cu") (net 2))
 (via (at 139.7 80.9) (size 0.6) (drill 0.3) (layers "F.Cu" "B.Cu") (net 2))
 (via (at 142.13125 71.76875) (size 0.6) (drill 0.3) (layers "F.Cu" "B.Cu") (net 2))
 (segment (start 140.649946 80.9) (end 139.7 80.9) (width 0.2) (layer "B.Cu") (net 2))
 (segment (start 142.13125 71.76875) (end 142.13125 79.26875) (width 0.2) (layer "B.Cu") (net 2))
 (segment (start 142.13125 79.418696) (end 140.649946 80.9) (width 0.2) (layer "B.Cu") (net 2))
 (segment (start 142.13125 79.26875) (end 142.13125 79.418696) (width 0.2) (layer "B.Cu") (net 2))
 (segment (start 141.906985 85.193015) (end 141.606985 85.193015) (width 0.2) (layer "F.Cu") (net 3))
 (segment (start 160.63125 78.16875) (end 150.73125 78.16875) (width 0.2) (layer "F.Cu") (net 3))
 (segment (start 139.775735 83.675735) (end 139.35147 84.1) (width 0.2) (layer "F.Cu") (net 3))
 (segment (start 125.3 84.9) (end 125.3 108.21) (width 0.2) (layer "F.Cu") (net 3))
 (segment (start 126.1 84.1) (end 125.3 84.9) (width 0.2) (layer "F.Cu") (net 3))
 (segment (start 139.35147 84.1) (end 126.1 84.1) (width 0.2) (layer "F.Cu") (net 3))
 (segment (start 125.3 108.21) (end 129.94 108.21) (width 0.2) (layer "F.Cu") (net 3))
 (segment (start 143 84.1) (end 141.906985 85.193015) (width 0.2) (layer "F.Cu") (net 3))
 (segment (start 150.73125 78.16875) (end 145.63125 83.26875) (width 0.2) (layer "F.Cu") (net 3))
 (segment (start 143.63125 83.46875) (end 143 84.1) (width 0.2) (layer "F.Cu") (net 3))
 (via (at 139.775735 83.675735) (size 0.6) (drill 0.3) (layers "F.Cu" "B.Cu") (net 3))
 (via (at 143.63125 83.46875) (size 0.6) (drill 0.3) (layers "F.Cu" "B.Cu") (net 3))
 (via (at 145.63125 83.26875) (size 0.6) (drill 0.3) (layers "F.Cu" "B.Cu") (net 3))
 (via (at 141.606985 85.193015) (size 0.6) (drill 0.3) (layers "F.Cu" "B.Cu") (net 3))
 (segment (start 141.606985 85.193015) (end 141.293015 85.193015) (width 0.2) (layer "B.Cu") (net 3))
 (segment (start 145.63125 83.26875) (end 145.43125 83.46875) (width 0.2) (layer "B.Cu") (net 3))
 (segment (start 145.43125 83.46875) (end 143.63125 83.46875) (width 0.2) (layer "B.Cu") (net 3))
 (segment (start 141.293015 85.193015) (end 139.775735 83.675735) (width 0.2) (layer "B.Cu") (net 3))
 (segment (start 151.17125 75.62875) (end 144.9 81.9) (width 0.2) (layer "F.Cu") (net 4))
 (segment (start 144.9 108.21) (end 148.99 108.21) (width 0.2) (layer "F.Cu") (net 4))
 (segment (start 144.9 81.9) (end 144.9 108.21) (width 0.2) (layer "F.Cu") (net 4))
 (segment (start 159.79625 75.62875) (end 151.17125 75.62875) (width 0.2) (layer "F.Cu") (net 4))
 (segment (start 159.79625 73.08875) (end 152.635705 73.08875) (width 0.2) (layer "F.Cu") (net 11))
 (segment (start 138.4 83.3) (end 109 83.3) (width 0.2) (layer "F.Cu") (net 11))
 (segment (start 107 89.16) (end 110.89 89.16) (width 0.2) (layer "F.Cu") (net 11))
 (segment (start 152.635705 73.08875) (end 144.255947 81.468508) (width 0.2) (layer "F.Cu") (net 11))
 (segment (start 109 83.3) (end 107 85.3) (width 0.2) (layer "F.Cu") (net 11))
 (segment (start 139.93125 81.76875) (end 138.4 83.3) (width 0.2) (layer "F.Cu") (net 11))
 (segment (start 107 85.3) (end 107 89.16) (width 0.2) (layer "F.Cu") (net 11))
 (via (at 139.93125 81.76875) (size 0.6) (drill 0.3) (layers "F.Cu" "B.Cu") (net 11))
 (via (at 144.255947 81.468508) (size 0.6) (drill 0.3) (layers "F.Cu" "B.Cu") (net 11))
 (segment (start 141.53125 83.36875) (end 142.355705 83.36875) (width 0.2) (layer "B.Cu") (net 11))
 (segment (start 139.93125 81.76875) (end 141.53125 83.36875) (width 0.2) (layer "B.Cu") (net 11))
 (segment (start 142.355705 83.36875) (end 144.255947 81.468508) (width 0.2) (layer "B.Cu") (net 11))
 (segment (start 126.2661 84.501) (end 125.8 84.9671) (width 0.2) (layer "F.Cu") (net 10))
 (segment (start 154.05125 70.54875) (end 159.79625 70.54875) (width 0.2) (layer "F.Cu") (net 10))
 (segment (start 142.23125 82.26875) (end 142.03125 82.26875) (width 0.2) (layer "F.Cu") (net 10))
 (segment (start 139.8 84.5) (end 139.51857 84.5) (width 0.2) (layer "F.Cu") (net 10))
 (segment (start 139.51757 84.501) (end 126.2661 84.501) (width 0.2) (layer "F.Cu") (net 10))
 (segment (start 140.376735 83.924678) (end 140.024678 84.276735) (width 0.2) (layer "F.Cu") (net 10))
 (segment (start 143.53125 80.96875) (end 143.63125 80.96875) (width 0.2) (layer "F.Cu") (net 10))
 (segment (start 125.8 89.16) (end 129.94 89.16) (width 0.2) (layer "F.Cu") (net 10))
 (segment (start 143.63125 80.96875) (end 154.05125 70.54875) (width 0.2) (layer "F.Cu") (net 10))
 (segment (start 139.51857 84.5) (end 139.51757 84.501) (width 0.2) (layer "F.Cu") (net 10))
 (segment (start 125.8 84.9671) (end 125.8 89.16) (width 0.2) (layer "F.Cu") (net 10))
 (segment (start 142.33125 82.16875) (end 142.23125 82.26875) (width 0.2) (layer "F.Cu") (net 10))
 (segment (start 140.023265 84.276735) (end 139.8 84.5) (width 0.2) (layer "F.Cu") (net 10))
 (segment (start 142.03125 82.26875) (end 140.376735 83.923265) (width 0.2) (layer "F.Cu") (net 10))
 (segment (start 140.024678 84.276735) (end 140.023265 84.276735) (width 0.2) (layer "F.Cu") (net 10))
 (segment (start 140.376735 83.923265) (end 140.376735 83.924678) (width 0.2) (layer "F.Cu") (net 10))
 (via (at 142.33125 82.16875) (size 0.6) (drill 0.3) (layers "F.Cu" "B.Cu") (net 10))
 (via (at 143.53125 80.96875) (size 0.6) (drill 0.3) (layers "F.Cu" "B.Cu") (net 10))
 (segment (start 142.33125 82.16875) (end 143.53125 80.96875) (width 0.2) (layer "B.Cu") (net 10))
 (segment (start 146.9 83) (end 147.4 83) (width 0.2) (layer "F.Cu") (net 8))
 (segment (start 148.99 89.16) (end 145.4 89.16) (width 0.2) (layer "F.Cu") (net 8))
 (segment (start 145.4 89.16) (end 145.4 84.5) (width 0.2) (layer "F.Cu") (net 8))
 (segment (start 145.4 84.5) (end 146.9 83) (width 0.2) (layer "F.Cu") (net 8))
 (via (at 147.4 83) (size 0.6) (drill 0.3) (layers "F.Cu" "B.Cu") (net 8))
 (segment (start 147.4 83) (end 144.55625 80.15625) (width 0.2) (layer "B.Cu") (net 8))
 (segment (start 144.55625 80.15625) (end 144.55625 78.16875) (width 0.2) (layer "B.Cu") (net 8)))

